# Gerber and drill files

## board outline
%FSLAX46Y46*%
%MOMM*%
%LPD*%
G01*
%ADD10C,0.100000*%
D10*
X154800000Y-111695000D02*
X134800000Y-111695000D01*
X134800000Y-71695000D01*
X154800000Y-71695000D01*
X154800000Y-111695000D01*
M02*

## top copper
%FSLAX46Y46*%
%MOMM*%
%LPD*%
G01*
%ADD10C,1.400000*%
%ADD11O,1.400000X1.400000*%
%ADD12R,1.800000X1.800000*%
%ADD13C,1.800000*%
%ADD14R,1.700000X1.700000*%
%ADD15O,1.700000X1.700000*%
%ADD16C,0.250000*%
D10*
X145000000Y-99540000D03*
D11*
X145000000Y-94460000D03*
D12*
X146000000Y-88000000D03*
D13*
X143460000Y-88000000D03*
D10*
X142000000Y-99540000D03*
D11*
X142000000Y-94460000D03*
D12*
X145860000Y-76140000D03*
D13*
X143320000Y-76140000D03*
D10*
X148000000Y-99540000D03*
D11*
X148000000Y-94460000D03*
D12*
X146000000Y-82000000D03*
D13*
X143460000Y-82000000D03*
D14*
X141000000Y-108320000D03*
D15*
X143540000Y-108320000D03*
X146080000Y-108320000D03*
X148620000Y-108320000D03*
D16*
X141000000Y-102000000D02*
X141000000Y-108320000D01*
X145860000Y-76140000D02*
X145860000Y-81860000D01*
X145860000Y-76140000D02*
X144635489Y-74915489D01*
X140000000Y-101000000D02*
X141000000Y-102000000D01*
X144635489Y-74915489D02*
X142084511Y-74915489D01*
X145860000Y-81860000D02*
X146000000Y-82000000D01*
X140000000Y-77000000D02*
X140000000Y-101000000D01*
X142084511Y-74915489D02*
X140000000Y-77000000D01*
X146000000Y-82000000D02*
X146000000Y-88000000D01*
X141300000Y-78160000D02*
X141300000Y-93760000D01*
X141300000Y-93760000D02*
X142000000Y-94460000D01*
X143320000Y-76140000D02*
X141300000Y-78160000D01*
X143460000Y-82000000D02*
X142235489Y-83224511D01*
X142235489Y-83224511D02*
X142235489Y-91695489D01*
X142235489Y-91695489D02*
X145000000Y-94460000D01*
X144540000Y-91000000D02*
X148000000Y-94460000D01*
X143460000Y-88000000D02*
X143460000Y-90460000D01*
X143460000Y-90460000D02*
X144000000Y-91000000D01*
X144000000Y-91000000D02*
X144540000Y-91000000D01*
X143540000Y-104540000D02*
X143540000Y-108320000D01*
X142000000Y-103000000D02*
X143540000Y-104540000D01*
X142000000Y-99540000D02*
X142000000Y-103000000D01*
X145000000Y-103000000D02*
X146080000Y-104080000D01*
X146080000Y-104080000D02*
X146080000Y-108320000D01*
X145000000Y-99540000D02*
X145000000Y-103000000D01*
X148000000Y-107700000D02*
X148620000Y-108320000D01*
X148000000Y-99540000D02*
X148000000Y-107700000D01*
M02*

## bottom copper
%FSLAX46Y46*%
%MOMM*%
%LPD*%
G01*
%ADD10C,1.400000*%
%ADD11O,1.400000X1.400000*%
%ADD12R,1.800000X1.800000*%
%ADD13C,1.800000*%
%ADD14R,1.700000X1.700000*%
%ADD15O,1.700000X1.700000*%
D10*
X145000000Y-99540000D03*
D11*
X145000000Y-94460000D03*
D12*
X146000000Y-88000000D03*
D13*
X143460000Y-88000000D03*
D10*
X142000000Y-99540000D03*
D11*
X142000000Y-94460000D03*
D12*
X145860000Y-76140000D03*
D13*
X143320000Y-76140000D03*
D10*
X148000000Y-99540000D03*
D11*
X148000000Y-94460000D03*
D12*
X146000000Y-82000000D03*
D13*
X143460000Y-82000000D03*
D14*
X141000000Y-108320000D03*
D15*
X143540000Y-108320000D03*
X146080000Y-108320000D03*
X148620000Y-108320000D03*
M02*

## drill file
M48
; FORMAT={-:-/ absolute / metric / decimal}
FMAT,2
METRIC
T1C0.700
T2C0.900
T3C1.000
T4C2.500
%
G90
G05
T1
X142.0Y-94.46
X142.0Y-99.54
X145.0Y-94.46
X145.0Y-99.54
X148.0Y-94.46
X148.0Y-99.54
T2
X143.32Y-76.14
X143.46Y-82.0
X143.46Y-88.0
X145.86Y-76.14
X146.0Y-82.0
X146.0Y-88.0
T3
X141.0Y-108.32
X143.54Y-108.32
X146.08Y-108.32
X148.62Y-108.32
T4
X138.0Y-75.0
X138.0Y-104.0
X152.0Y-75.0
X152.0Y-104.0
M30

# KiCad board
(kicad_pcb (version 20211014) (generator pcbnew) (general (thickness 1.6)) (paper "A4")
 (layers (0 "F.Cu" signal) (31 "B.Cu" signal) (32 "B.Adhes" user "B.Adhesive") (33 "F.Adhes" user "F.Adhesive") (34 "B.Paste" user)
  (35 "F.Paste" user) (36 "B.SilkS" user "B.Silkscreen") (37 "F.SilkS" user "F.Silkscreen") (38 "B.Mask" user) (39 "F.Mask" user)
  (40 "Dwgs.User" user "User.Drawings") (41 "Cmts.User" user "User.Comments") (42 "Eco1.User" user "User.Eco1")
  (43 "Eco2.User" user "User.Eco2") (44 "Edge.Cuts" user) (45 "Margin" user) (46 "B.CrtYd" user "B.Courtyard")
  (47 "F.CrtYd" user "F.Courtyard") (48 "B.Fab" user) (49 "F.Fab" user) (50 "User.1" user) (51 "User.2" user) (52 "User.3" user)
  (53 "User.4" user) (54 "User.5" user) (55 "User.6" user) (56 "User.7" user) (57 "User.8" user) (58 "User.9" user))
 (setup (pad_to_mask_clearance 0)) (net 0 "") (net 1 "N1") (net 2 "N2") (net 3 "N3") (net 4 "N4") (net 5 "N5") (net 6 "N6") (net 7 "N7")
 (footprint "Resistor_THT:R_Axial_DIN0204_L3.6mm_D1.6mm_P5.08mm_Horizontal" (layer "F.Cu") (at 145 99.54 90)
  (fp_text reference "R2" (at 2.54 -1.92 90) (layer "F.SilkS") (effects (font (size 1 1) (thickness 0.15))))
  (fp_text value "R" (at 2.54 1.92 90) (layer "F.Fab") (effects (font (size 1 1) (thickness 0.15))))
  (pad "1" thru_hole circle (at 0 0 90) (size 1.4 1.4) (drill 0.7) (layers *.Cu *.Mask) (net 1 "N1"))
  (pad "2" thru_hole oval (at 5.08 0 90) (size 1.4 1.4) (drill 0.7) (layers *.Cu *.Mask) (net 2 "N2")))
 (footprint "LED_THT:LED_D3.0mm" (layer "F.Cu") (at 146 88 180)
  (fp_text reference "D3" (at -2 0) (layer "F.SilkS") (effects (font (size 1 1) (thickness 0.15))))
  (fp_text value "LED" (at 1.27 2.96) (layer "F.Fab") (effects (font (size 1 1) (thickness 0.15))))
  (pad "1" thru_hole rect (at 0 0 180) (size 1.8 1.8) (drill 0.9) (layers *.Cu *.Mask) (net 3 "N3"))
  (pad "2" thru_hole circle (at 2.54 0 180) (size 1.8 1.8) (drill 0.9) (layers *.Cu *.Mask) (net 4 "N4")))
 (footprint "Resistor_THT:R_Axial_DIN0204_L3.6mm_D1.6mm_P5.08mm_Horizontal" (layer "F.Cu") (at 142 99.54 90)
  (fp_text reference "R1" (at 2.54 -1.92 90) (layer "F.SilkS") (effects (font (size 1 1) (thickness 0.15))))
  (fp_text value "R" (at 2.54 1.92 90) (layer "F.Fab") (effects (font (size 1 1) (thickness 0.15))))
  (pad "1" thru_hole circle (at 0 0 90) (size 1.4 1.4) (drill 0.7) (layers *.Cu *.Mask) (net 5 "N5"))
  (pad "2" thru_hole oval (at 5.08 0 90) (size 1.4 1.4) (drill 0.7) (layers *.Cu *.Mask) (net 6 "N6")))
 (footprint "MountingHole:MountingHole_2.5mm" (layer "F.Cu") (at 152 75)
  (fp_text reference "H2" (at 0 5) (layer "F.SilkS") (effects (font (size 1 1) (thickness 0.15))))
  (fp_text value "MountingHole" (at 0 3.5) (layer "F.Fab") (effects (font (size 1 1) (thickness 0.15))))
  (pad "" np_thru_hole circle (at 0 0) (size 2.5 2.5) (drill 2.5) (layers *.Cu *.Mask)))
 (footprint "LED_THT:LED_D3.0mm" (layer "F.Cu") (at 145.86 76.14 180)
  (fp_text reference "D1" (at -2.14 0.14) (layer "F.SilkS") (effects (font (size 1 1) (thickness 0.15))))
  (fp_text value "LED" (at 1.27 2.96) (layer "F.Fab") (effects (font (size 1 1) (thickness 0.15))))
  (pad "1" thru_hole rect (at 0 0 180) (size 1.8 1.8) (drill 0.9) (layers *.Cu *.Mask) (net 3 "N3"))
  (pad "2" thru_hole circle (at 2.54 0 180) (size 1.8 1.8) (drill 0.9) (layers *.Cu *.Mask) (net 6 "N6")))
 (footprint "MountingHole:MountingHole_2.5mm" (layer "F.Cu") (at 138 104)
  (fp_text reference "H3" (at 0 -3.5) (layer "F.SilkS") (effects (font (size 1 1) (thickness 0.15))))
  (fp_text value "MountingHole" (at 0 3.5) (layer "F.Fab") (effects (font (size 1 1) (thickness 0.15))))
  (pad "" np_thru_hole circle (at 0 0) (size 2.5 2.5) (drill 2.5) (layers *.Cu *.Mask)))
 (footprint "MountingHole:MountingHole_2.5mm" (layer "F.Cu") (at 152 104)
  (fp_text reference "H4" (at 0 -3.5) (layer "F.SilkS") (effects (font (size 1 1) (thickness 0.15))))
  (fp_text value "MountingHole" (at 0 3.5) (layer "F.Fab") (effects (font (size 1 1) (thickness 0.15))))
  (pad "" np_thru_hole circle (at 0 0) (size 2.5 2.5) (drill 2.5) (layers *.Cu *.Mask)))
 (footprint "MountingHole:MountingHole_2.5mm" (layer "F.Cu") (at 138 75)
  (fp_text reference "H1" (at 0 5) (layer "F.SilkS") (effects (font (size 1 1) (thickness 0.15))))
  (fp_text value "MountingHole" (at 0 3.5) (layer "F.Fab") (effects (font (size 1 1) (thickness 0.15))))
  (pad "" np_thru_hole circle (at 0 0) (size 2.5 2.5) (drill 2.5) (layers *.Cu *.Mask)))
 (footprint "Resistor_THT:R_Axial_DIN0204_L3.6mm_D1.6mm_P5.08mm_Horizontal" (layer "F.Cu") (at 148 99.54 90)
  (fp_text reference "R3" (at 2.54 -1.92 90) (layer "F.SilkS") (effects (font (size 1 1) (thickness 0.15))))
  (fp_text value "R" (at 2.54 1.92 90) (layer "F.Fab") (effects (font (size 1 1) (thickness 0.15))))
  (pad "1" thru_hole circle (at 0 0 90) (size 1.4 1.4) (drill 0.7) (layers *.Cu *.Mask) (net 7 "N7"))
  (pad "2" thru_hole oval (at 5.08 0 90) (size 1.4 1.4) (drill 0.7) (layers *.Cu *.Mask) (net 4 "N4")))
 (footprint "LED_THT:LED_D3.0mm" (layer "F.Cu") (at 146 82 180)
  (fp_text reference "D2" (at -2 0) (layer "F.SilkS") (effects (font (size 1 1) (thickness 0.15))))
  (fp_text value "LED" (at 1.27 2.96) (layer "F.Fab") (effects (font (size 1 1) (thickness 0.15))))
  (pad "1" thru_hole rect (at 0 0 180) (size 1.8 1.8) (drill 0.9) (layers *.Cu *.Mask) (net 3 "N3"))
  (pad "2" thru_hole circle (at 2.54 0 180) (size 1.8 1.8) (drill 0.9) (layers *.Cu *.Mask) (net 2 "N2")))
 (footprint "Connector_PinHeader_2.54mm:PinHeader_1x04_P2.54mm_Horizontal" (layer "B.Cu") (at 141 108.32 -90)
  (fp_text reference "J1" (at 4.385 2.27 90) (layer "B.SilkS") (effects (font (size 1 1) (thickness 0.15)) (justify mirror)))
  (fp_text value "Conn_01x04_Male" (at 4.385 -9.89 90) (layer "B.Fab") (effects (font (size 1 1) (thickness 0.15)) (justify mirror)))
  (pad "1" thru_hole rect (at 0 0 270) (size 1.7 1.7) (drill 1) (layers *.Cu *.Mask) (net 3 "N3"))
  (pad "2" thru_hole oval (at 0 -2.54 270) (size 1.7 1.7) (drill 1) (layers *.Cu *.Mask) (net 5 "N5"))
  (pad "3" thru_hole oval (at 0 -5.08 270) (size 1.7 1.7) (drill 1) (layers *.Cu *.Mask) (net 1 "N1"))
  (pad "4" thru_hole oval (at 0 -7.62 270) (size 1.7 1.7) (drill 1) (layers *.Cu *.Mask) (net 7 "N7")))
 (gr_poly (pts (xy 154.8 111.695) (xy 134.8 111.695) (xy 134.8 71.695) (xy 154.8 71.695)) (layer "Edge.Cuts") (width 0.1) (fill none))
 (segment (start 141 102) (end 141 108.32) (width 0.25) (layer "F.Cu") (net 3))
 (segment (start 145.86 76.14) (end 145.86 81.86) (width 0.25) (layer "F.Cu") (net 3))
 (segment (start 145.86 76.14) (end 144.635489 74.915489) (width 0.25) (layer "F.Cu") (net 3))
 (segment (start 140 101) (end 141 102) (width 0.25) (layer "F.Cu") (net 3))
 (segment (start 144.635489 74.915489) (end 142.084511 74.915489) (width 0.25) (layer "F.Cu") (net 3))
 (segment (start 145.86 81.86) (end 146 82) (width 0.25) (layer "F.Cu") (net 3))
 (segment (start 140 77) (end 140 101) (width 0.25) (layer "F.Cu") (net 3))
 (segment (start 142.084511 74.915489) (end 140 77) (width 0.25) (layer "F.Cu") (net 3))
 (segment (start 146 82) (end 146 88) (width 0.25) (layer "F.Cu") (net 3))
 (segment (start 141.3 78.16) (end 141.3 93.76) (width 0.25) (layer "F.Cu") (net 6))
 (segment (start 141.3 93.76) (end 142 94.46) (width 0.25) (layer "F.Cu") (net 6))
 (segment (start 143.32 76.14) (end 141.3 78.16) (width 0.25) (layer "F.Cu") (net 6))
 (segment (start 143.46 82) (end 142.235489 83.224511) (width 0.25) (layer "F.Cu") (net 2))
 (segment (start 142.235489 83.224511) (end 142.235489 91.695489) (width 0.25) (layer "F.Cu") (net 2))
 (segment (start 142.235489 91.695489) (end 145 94.46) (width 0.25) (layer "F.Cu") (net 2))
 (segment (start 144.54 91) (end 148 94.46) (width 0.25) (layer "F.Cu") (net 4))
 (segment (start 143.46 88) (end 143.46 90.46) (width 0.25) (layer "F.Cu") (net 4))
 (segment (start 143.46 90.46) (end 144 91) (width 0.25) (layer "F.Cu") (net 4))
 (segment (start 144 91) (end 144.54 91) (width 0.25) (layer "F.Cu") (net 4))
 (segment (start 143.54 104.54) (end 143.54 108.32) (width 0.25) (layer "F.Cu") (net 5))
 (segment (start 142 103) (end 143.54 104.54) (width 0.25) (layer "F.Cu") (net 5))
 (segment (start 142 99.54) (end 142 103) (width 0.25) (layer "F.Cu") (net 5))
 (segment (start 145 103) (end 146.08 104.08) (width 0.25) (layer "F.Cu") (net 1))
 (segment (start 146.08 104.08) (end 146.08 108.32) (width 0.25) (layer "F.Cu") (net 1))
 (segment (start 145 99.54) (end 145 103) (width 0.25) (layer "F.Cu") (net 1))
 (segment (start 148 107.7) (end 148.62 108.32) (width 0.25) (layer "F.Cu") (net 7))
 (segment (start 148 99.54) (end 148 107.7) (width 0.25) (layer "F.Cu") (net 7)))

